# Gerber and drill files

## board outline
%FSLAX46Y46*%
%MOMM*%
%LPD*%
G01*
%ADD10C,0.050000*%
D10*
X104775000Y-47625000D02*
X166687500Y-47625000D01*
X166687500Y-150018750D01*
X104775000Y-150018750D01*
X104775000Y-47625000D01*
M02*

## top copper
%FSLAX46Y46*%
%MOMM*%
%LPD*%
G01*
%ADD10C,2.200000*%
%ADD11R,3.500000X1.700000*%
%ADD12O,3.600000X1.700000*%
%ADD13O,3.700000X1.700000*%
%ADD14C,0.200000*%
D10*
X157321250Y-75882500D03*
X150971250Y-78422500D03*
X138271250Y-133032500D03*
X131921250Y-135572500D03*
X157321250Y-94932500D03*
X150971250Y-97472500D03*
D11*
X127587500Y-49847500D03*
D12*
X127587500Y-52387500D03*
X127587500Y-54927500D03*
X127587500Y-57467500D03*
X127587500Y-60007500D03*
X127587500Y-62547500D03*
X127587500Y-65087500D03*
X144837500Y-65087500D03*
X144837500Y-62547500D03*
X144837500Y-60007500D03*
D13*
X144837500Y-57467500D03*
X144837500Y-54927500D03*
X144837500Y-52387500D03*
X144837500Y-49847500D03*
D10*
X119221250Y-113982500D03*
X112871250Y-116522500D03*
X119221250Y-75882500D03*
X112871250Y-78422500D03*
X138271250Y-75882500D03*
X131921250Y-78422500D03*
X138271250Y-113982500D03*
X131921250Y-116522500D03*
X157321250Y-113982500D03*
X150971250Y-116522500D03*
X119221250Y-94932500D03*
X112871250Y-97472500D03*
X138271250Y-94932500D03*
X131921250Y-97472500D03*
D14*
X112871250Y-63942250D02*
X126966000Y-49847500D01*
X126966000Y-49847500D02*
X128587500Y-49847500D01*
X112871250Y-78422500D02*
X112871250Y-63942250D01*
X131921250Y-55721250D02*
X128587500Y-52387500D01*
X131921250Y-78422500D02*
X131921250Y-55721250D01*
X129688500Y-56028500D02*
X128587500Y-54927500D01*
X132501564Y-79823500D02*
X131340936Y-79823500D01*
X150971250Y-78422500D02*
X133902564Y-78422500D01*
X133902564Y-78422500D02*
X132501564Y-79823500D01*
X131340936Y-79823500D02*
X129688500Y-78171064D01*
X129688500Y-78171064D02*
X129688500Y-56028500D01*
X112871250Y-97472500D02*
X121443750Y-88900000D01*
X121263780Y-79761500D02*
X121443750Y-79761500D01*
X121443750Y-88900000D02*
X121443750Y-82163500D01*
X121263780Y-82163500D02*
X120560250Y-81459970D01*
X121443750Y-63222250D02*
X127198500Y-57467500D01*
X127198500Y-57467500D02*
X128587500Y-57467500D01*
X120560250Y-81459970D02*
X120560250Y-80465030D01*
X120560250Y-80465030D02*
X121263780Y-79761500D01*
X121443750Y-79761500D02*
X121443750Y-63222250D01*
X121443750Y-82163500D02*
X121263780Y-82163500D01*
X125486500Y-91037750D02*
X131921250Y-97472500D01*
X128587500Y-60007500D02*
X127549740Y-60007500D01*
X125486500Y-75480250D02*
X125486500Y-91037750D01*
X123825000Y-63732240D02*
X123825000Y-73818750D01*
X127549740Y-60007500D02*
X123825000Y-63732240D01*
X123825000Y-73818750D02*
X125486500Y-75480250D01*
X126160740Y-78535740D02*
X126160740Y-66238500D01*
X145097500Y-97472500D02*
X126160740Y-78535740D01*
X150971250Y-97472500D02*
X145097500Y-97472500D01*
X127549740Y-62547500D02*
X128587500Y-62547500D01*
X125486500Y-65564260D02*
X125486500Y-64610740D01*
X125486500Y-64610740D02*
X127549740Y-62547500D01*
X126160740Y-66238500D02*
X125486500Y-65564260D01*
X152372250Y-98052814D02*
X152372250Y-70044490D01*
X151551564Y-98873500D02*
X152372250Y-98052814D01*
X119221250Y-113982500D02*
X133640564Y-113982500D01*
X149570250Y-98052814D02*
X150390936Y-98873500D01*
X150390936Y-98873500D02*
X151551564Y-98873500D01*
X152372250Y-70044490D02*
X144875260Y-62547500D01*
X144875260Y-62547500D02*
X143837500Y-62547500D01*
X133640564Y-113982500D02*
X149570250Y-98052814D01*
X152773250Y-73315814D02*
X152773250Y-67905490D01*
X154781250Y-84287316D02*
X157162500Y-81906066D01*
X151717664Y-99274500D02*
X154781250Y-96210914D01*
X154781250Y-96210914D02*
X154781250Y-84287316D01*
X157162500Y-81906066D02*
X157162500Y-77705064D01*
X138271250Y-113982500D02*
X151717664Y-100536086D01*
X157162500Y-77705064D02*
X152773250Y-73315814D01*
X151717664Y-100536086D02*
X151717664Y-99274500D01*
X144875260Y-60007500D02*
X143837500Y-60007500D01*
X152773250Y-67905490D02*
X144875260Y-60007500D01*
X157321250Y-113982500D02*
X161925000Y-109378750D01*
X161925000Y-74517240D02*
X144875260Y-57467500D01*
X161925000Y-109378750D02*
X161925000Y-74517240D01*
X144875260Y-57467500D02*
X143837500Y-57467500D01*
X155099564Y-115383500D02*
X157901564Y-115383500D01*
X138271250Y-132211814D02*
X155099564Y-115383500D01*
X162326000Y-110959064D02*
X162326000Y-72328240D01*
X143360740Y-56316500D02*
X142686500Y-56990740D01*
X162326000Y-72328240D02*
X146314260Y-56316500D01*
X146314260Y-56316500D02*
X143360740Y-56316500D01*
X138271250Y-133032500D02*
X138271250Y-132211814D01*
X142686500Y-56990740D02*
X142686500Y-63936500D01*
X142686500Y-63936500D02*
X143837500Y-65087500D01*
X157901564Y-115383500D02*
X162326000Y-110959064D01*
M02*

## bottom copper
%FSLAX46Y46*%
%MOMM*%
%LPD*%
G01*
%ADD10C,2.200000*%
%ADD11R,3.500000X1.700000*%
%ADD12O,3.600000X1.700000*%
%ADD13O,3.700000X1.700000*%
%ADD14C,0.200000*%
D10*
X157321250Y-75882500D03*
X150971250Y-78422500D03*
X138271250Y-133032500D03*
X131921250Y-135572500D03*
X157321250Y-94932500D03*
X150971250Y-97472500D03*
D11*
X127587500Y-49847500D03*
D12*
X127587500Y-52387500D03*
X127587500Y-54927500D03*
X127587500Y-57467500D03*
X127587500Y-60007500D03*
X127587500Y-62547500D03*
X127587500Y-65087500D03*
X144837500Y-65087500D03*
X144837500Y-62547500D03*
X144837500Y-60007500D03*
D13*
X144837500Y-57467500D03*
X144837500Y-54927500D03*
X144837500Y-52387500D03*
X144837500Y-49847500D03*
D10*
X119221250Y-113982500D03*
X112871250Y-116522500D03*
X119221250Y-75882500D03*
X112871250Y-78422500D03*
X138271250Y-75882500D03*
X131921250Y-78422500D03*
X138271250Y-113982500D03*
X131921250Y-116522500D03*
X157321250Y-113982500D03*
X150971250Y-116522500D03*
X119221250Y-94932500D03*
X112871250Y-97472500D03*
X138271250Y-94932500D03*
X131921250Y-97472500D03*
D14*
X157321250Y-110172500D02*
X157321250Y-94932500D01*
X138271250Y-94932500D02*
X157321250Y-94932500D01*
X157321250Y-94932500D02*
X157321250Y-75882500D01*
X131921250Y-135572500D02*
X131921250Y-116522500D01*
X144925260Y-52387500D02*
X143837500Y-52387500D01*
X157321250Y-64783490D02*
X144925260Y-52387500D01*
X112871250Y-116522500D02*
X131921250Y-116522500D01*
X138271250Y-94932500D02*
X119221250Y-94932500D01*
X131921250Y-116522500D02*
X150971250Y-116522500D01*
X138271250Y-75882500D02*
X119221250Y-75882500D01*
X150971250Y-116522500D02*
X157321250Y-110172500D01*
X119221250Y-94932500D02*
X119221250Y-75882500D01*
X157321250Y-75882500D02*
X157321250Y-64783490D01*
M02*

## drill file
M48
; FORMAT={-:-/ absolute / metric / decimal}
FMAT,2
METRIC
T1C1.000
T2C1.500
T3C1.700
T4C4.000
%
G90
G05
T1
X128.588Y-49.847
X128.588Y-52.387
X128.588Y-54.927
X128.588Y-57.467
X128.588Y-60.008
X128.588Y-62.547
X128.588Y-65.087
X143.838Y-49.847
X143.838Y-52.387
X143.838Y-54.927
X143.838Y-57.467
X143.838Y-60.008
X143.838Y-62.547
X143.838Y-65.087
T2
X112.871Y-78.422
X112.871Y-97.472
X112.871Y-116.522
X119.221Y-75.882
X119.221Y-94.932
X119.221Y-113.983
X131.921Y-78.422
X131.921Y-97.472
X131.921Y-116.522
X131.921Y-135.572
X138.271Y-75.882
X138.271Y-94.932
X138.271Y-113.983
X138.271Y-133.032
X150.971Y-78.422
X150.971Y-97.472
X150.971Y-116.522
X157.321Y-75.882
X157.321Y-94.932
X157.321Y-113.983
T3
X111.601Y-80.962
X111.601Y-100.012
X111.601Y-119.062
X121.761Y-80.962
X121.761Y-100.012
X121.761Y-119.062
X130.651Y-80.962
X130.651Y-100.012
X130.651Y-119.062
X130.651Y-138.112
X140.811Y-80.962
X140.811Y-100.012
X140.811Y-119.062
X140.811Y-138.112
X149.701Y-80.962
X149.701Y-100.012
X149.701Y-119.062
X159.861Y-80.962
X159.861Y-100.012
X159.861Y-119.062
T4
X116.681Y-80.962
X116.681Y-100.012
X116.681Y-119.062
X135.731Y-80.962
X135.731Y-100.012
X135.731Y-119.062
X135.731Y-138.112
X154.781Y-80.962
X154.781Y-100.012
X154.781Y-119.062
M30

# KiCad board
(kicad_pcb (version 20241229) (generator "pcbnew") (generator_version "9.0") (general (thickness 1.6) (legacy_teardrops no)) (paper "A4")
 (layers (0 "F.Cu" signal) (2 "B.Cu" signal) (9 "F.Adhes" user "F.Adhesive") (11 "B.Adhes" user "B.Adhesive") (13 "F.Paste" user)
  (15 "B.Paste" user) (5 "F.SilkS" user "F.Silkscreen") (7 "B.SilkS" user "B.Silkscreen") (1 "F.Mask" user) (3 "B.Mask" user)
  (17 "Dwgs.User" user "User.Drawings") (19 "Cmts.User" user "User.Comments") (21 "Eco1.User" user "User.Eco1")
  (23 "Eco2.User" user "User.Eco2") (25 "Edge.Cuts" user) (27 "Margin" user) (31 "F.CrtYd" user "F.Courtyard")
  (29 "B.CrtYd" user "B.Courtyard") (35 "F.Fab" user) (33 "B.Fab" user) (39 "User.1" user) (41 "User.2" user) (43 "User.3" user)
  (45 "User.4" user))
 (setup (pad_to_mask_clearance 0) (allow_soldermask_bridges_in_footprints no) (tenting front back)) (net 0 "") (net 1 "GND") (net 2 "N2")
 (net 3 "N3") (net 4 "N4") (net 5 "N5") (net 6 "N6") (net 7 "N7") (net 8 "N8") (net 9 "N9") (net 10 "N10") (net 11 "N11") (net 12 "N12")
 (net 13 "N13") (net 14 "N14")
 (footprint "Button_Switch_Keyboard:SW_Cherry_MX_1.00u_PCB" (layer "F.Cu") (at 157.32125 75.8825)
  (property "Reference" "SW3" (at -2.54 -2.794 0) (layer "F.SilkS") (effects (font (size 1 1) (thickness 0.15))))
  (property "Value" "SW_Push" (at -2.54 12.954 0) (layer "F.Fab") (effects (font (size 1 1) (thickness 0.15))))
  (pad "" np_thru_hole circle (at -7.62 5.08) (size 1.7 1.7) (drill 1.7) (layers "*.Cu" "*.Mask"))
  (pad "" np_thru_hole circle (at -2.54 5.08) (size 4 4) (drill 4) (layers "*.Cu" "*.Mask"))
  (pad "" np_thru_hole circle (at 2.54 5.08) (size 1.7 1.7) (drill 1.7) (layers "*.Cu" "*.Mask"))
  (pad "1" thru_hole circle (at 0 0) (size 2.2 2.2) (drill 1.5) (layers "*.Cu" "*.Mask") (remove_unused_layers no) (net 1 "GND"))
  (pad "2" thru_hole circle (at -6.35 2.54) (size 2.2 2.2) (drill 1.5) (layers "*.Cu" "*.Mask") (remove_unused_layers no) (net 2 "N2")))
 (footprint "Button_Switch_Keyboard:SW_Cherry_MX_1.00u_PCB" (layer "F.Cu") (at 138.27125 133.0325)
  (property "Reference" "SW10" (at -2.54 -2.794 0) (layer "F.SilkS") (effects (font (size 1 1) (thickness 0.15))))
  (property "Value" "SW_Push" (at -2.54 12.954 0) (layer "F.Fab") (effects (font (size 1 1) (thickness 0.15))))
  (pad "" np_thru_hole circle (at -7.62 5.08) (size 1.7 1.7) (drill 1.7) (layers "*.Cu" "*.Mask"))
  (pad "" np_thru_hole circle (at -2.54 5.08) (size 4 4) (drill 4) (layers "*.Cu" "*.Mask"))
  (pad "" np_thru_hole circle (at 2.54 5.08) (size 1.7 1.7) (drill 1.7) (layers "*.Cu" "*.Mask"))
  (pad "1" thru_hole circle (at 0 0) (size 2.2 2.2) (drill 1.5) (layers "*.Cu" "*.Mask") (remove_unused_layers no) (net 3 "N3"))
  (pad "2" thru_hole circle (at -6.35 2.54) (size 2.2 2.2) (drill 1.5) (layers "*.Cu" "*.Mask") (remove_unused_layers no) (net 1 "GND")))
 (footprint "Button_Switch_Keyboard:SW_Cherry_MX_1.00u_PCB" (layer "F.Cu") (at 157.32125 94.9325)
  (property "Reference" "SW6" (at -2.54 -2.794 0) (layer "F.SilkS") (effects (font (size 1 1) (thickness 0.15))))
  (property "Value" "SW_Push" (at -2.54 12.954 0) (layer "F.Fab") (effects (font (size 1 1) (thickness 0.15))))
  (pad "" np_thru_hole circle (at -7.62 5.08) (size 1.7 1.7) (drill 1.7) (layers "*.Cu" "*.Mask"))
  (pad "" np_thru_hole circle (at -2.54 5.08) (size 4 4) (drill 4) (layers "*.Cu" "*.Mask"))
  (pad "" np_thru_hole circle (at 2.54 5.08) (size 1.7 1.7) (drill 1.7) (layers "*.Cu" "*.Mask"))
  (pad "1" thru_hole circle (at 0 0) (size 2.2 2.2) (drill 1.5) (layers "*.Cu" "*.Mask") (remove_unused_layers no) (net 1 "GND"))
  (pad "2" thru_hole circle (at -6.35 2.54) (size 2.2 2.2) (drill 1.5) (layers "*.Cu" "*.Mask") (remove_unused_layers no) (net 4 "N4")))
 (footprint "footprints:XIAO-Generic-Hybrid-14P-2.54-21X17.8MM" (layer "F.Cu") (at 136.2125 57.4675)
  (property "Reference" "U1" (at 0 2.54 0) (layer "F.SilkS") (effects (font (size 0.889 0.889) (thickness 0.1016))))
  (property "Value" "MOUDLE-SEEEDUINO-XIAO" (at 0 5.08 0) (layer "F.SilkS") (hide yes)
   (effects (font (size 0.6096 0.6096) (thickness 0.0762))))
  (pad "1" thru_hole rect (at -7.625 -7.62) (size 3.5 1.7) (drill 1 (offset -1 0)) (layers "*.Cu" "*.Mask") (remove_unused_layers no)
   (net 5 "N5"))
  (pad "2" thru_hole oval (at -7.625 -5.08) (size 3.6 1.7) (drill 1 (offset -1 0)) (layers "*.Cu" "*.Mask") (remove_unused_layers no)
   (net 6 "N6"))
  (pad "3" thru_hole oval (at -7.625 -2.54) (size 3.6 1.7) (drill 1 (offset -1 0)) (layers "*.Cu" "*.Mask") (remove_unused_layers no)
   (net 2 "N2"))
  (pad "4" thru_hole oval (at -7.625 0) (size 3.6 1.7) (drill 1 (offset -1 0)) (layers "*.Cu" "*.Mask") (remove_unused_layers no)
   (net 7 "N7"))
  (pad "5" thru_hole oval (at -7.625 2.54) (size 3.6 1.7) (drill 1 (offset -1 0)) (layers "*.Cu" "*.Mask") (remove_unused_layers no)
   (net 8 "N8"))
  (pad "6" thru_hole oval (at -7.625 5.08 180) (size 3.6 1.7) (drill 1 (offset 1 0)) (layers "*.Cu" "*.Mask") (remove_unused_layers no)
   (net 4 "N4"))
  (pad "7" thru_hole oval (at -7.625 7.62) (size 3.6 1.7) (drill 1 (offset -1 0)) (layers "*.Cu" "*.Mask") (remove_unused_layers no)
   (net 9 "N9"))
  (pad "8" thru_hole oval (at 7.625 7.62) (size 3.6 1.7) (drill 1 (offset 1 0)) (layers "*.Cu" "*.Mask") (remove_unused_layers no)
   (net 3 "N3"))
  (pad "9" thru_hole oval (at 7.625 5.08) (size 3.6 1.7) (drill 1 (offset 1 0)) (layers "*.Cu" "*.Mask") (remove_unused_layers no)
   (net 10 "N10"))
  (pad "10" thru_hole oval (at 7.625 2.54) (size 3.6 1.7) (drill 1 (offset 1 0)) (layers "*.Cu" "*.Mask") (remove_unused_layers no)
   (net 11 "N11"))
  (pad "11" thru_hole oval (at 7.625 0) (size 3.7 1.7) (drill 1 (offset 1 0)) (layers "*.Cu" "*.Mask") (remove_unused_layers no)
   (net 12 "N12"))
  (pad "12" thru_hole oval (at 7.625 -2.54) (size 3.7 1.7) (drill 1 (offset 1 0)) (layers "*.Cu" "*.Mask") (remove_unused_layers no)
   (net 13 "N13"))
  (pad "13" thru_hole oval (at 7.625 -5.08) (size 3.7 1.7) (drill 1 (offset 1 0)) (layers "*.Cu" "*.Mask") (remove_unused_layers no)
   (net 1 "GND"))
  (pad "14" thru_hole oval (at 7.625 -7.62) (size 3.7 1.7) (drill 1 (offset 1 0)) (layers "*.Cu" "*.Mask") (remove_unused_layers no)
   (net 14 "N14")))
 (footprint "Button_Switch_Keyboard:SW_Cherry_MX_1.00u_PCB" (layer "F.Cu") (at 119.22125 113.9825)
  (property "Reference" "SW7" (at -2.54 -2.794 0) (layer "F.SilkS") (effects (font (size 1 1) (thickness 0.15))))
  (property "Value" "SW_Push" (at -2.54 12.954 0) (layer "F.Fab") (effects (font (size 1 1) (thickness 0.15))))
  (pad "" np_thru_hole circle (at -7.62 5.08) (size 1.7 1.7) (drill 1.7) (layers "*.Cu" "*.Mask"))
  (pad "" np_thru_hole circle (at -2.54 5.08) (size 4 4) (drill 4) (layers "*.Cu" "*.Mask"))
  (pad "" np_thru_hole circle (at 2.54 5.08) (size 1.7 1.7) (drill 1.7) (layers "*.Cu" "*.Mask"))
  (pad "1" thru_hole circle (at 0 0) (size 2.2 2.2) (drill 1.5) (layers "*.Cu" "*.Mask") (remove_unused_layers no) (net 10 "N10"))
  (pad "2" thru_hole circle (at -6.35 2.54) (size 2.2 2.2) (drill 1.5) (layers "*.Cu" "*.Mask") (remove_unused_layers no) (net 1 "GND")))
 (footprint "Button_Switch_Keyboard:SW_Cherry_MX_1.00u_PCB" (layer "F.Cu") (at 119.22125 75.8825)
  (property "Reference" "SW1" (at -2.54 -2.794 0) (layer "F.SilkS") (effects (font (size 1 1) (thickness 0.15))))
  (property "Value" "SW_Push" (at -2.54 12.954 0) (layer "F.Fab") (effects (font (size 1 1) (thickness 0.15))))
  (pad "" np_thru_hole circle (at -7.62 5.08) (size 1.7 1.7) (drill 1.7) (layers "*.Cu" "*.Mask"))
  (pad "" np_thru_hole circle (at -2.54 5.08) (size 4 4) (drill 4) (layers "*.Cu" "*.Mask"))
  (pad "" np_thru_hole circle (at 2.54 5.08) (size 1.7 1.7) (drill 1.7) (layers "*.Cu" "*.Mask"))
  (pad "1" thru_hole circle (at 0 0) (size 2.2 2.2) (drill 1.5) (layers "*.Cu" "*.Mask") (remove_unused_layers no) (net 1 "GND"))
  (pad "2" thru_hole circle (at -6.35 2.54) (size 2.2 2.2) (drill 1.5) (layers "*.Cu" "*.Mask") (remove_unused_layers no) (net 5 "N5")))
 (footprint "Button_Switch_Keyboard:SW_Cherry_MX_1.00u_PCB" (layer "F.Cu") (at 138.27125 75.8825)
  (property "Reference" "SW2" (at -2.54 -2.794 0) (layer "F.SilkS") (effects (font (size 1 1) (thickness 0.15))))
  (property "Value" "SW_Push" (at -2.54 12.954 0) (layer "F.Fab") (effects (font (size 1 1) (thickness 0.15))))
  (pad "" np_thru_hole circle (at -7.62 5.08) (size 1.7 1.7) (drill 1.7) (layers "*.Cu" "*.Mask"))
  (pad "" np_thru_hole circle (at -2.54 5.08) (size 4 4) (drill 4) (layers "*.Cu" "*.Mask"))
  (pad "" np_thru_hole circle (at 2.54 5.08) (size 1.7 1.7) (drill 1.7) (layers "*.Cu" "*.Mask"))
  (pad "1" thru_hole circle (at 0 0) (size 2.2 2.2) (drill 1.5) (layers "*.Cu" "*.Mask") (remove_unused_layers no) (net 1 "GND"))
  (pad "2" thru_hole circle (at -6.35 2.54) (size 2.2 2.2) (drill 1.5) (layers "*.Cu" "*.Mask") (remove_unused_layers no) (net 6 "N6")))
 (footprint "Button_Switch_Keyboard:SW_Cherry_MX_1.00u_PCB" (layer "F.Cu") (at 138.27125 113.9825)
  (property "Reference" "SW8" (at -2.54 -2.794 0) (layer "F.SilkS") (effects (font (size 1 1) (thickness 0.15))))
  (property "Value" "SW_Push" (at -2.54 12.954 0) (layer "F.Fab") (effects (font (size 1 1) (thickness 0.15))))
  (pad "" np_thru_hole circle (at -7.62 5.08) (size 1.7 1.7) (drill 1.7) (layers "*.Cu" "*.Mask"))
  (pad "" np_thru_hole circle (at -2.54 5.08) (size 4 4) (drill 4) (layers "*.Cu" "*.Mask"))
  (pad "" np_thru_hole circle (at 2.54 5.08) (size 1.7 1.7) (drill 1.7) (layers "*.Cu" "*.Mask"))
  (pad "1" thru_hole circle (at 0 0) (size 2.2 2.2) (drill 1.5) (layers "*.Cu" "*.Mask") (remove_unused_layers no) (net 11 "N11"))
  (pad "2" thru_hole circle (at -6.35 2.54) (size 2.2 2.2) (drill 1.5) (layers "*.Cu" "*.Mask") (remove_unused_layers no) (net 1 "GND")))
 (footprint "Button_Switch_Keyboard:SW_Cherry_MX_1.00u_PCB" (layer "F.Cu") (at 157.32125 113.9825)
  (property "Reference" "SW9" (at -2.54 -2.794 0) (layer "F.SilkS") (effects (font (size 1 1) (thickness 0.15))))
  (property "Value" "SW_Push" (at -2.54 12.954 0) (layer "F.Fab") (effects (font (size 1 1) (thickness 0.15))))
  (pad "" np_thru_hole circle (at -7.62 5.08) (size 1.7 1.7) (drill 1.7) (layers "*.Cu" "*.Mask"))
  (pad "" np_thru_hole circle (at -2.54 5.08) (size 4 4) (drill 4) (layers "*.Cu" "*.Mask"))
  (pad "" np_thru_hole circle (at 2.54 5.08) (size 1.7 1.7) (drill 1.7) (layers "*.Cu" "*.Mask"))
  (pad "1" thru_hole circle (at 0 0) (size 2.2 2.2) (drill 1.5) (layers "*.Cu" "*.Mask") (remove_unused_layers no) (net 12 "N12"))
  (pad "2" thru_hole circle (at -6.35 2.54) (size 2.2 2.2) (drill 1.5) (layers "*.Cu" "*.Mask") (remove_unused_layers no) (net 1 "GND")))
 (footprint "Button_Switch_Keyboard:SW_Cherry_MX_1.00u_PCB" (layer "F.Cu") (at 119.22125 94.9325)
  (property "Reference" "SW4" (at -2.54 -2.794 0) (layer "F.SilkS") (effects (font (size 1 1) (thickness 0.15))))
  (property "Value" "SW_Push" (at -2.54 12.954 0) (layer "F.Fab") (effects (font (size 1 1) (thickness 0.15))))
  (pad "" np_thru_hole circle (at -7.62 5.08) (size 1.7 1.7) (drill 1.7) (layers "*.Cu" "*.Mask"))
  (pad "" np_thru_hole circle (at -2.54 5.08) (size 4 4) (drill 4) (layers "*.Cu" "*.Mask"))
  (pad "" np_thru_hole circle (at 2.54 5.08) (size 1.7 1.7) (drill 1.7) (layers "*.Cu" "*.Mask"))
  (pad "1" thru_hole circle (at 0 0) (size 2.2 2.2) (drill 1.5) (layers "*.Cu" "*.Mask") (remove_unused_layers no) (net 1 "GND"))
  (pad "2" thru_hole circle (at -6.35 2.54) (size 2.2 2.2) (drill 1.5) (layers "*.Cu" "*.Mask") (remove_unused_layers no) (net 7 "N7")))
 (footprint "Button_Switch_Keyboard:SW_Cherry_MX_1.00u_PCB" (layer "F.Cu") (at 138.27125 94.9325)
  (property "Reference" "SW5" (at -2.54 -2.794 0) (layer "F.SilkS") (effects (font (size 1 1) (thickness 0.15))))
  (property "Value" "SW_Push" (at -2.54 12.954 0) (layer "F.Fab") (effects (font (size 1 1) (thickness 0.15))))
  (pad "" np_thru_hole circle (at -7.62 5.08) (size 1.7 1.7) (drill 1.7) (layers "*.Cu" "*.Mask"))
  (pad "" np_thru_hole circle (at -2.54 5.08) (size 4 4) (drill 4) (layers "*.Cu" "*.Mask"))
  (pad "" np_thru_hole circle (at 2.54 5.08) (size 1.7 1.7) (drill 1.7) (layers "*.Cu" "*.Mask"))
  (pad "1" thru_hole circle (at 0 0) (size 2.2 2.2) (drill 1.5) (layers "*.Cu" "*.Mask") (remove_unused_layers no) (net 1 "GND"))
  (pad "2" thru_hole circle (at -6.35 2.54) (size 2.2 2.2) (drill 1.5) (layers "*.Cu" "*.Mask") (remove_unused_layers no) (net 8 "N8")))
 (gr_rect (start 104.775 47.625) (end 166.6875 150.01875) (stroke (width 0.05) (type default)) (fill no) (layer "Edge.Cuts"))
 (segment (start 112.87125 63.94225) (end 126.966 49.8475) (width 0.2) (layer "F.Cu") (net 5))
 (segment (start 126.966 49.8475) (end 128.5875 49.8475) (width 0.2) (layer "F.Cu") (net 5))
 (segment (start 112.87125 78.4225) (end 112.87125 63.94225) (width 0.2) (layer "F.Cu") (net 5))
 (segment (start 157.32125 110.1725) (end 157.32125 94.9325) (width 0.2) (layer "B.Cu") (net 1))
 (segment (start 138.27125 94.9325) (end 157.32125 94.9325) (width 0.2) (layer "B.Cu") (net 1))
 (segment (start 157.32125 94.9325) (end 157.32125 75.8825) (width 0.2) (layer "B.Cu") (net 1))
 (segment (start 131.92125 135.5725) (end 131.92125 116.5225) (width 0.2) (layer "B.Cu") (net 1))
 (segment (start 144.92526 52.3875) (end 143.8375 52.3875) (width 0.2) (layer "B.Cu") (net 1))
 (segment (start 157.32125 64.78349) (end 144.92526 52.3875) (width 0.2) (layer "B.Cu") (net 1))
 (segment (start 112.87125 116.5225) (end 131.92125 116.5225) (width 0.2) (layer "B.Cu") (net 1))
 (segment (start 138.27125 94.9325) (end 119.22125 94.9325) (width 0.2) (layer "B.Cu") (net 1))
 (segment (start 131.92125 116.5225) (end 150.97125 116.5225) (width 0.2) (layer "B.Cu") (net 1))
 (segment (start 138.27125 75.8825) (end 119.22125 75.8825) (width 0.2) (layer "B.Cu") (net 1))
 (segment (start 150.97125 116.5225) (end 157.32125 110.1725) (width 0.2) (layer "B.Cu") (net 1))
 (segment (start 119.22125 94.9325) (end 119.22125 75.8825) (width 0.2) (layer "B.Cu") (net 1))
 (segment (start 157.32125 75.8825) (end 157.32125 64.78349) (width 0.2) (layer "B.Cu") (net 1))
 (segment (start 131.92125 55.72125) (end 128.5875 52.3875) (width 0.2) (layer "F.Cu") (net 6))
 (segment (start 131.92125 78.4225) (end 131.92125 55.72125) (width 0.2) (layer "F.Cu") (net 6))
 (segment (start 129.6885 56.0285) (end 128.5875 54.9275) (width 0.2) (layer "F.Cu") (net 2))
 (segment (start 132.501564 79.8235) (end 131.340936 79.8235) (width 0.2) (layer "F.Cu") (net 2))
 (segment (start 150.97125 78.4225) (end 133.902564 78.4225) (width 0.2) (layer "F.Cu") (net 2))
 (segment (start 133.902564 78.4225) (end 132.501564 79.8235) (width 0.2) (layer "F.Cu") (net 2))
 (segment (start 131.340936 79.8235) (end 129.6885 78.171064) (width 0.2) (layer "F.Cu") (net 2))
 (segment (start 129.6885 78.171064) (end 129.6885 56.0285) (width 0.2) (layer "F.Cu") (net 2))
 (segment (start 112.87125 97.4725) (end 121.44375 88.9) (width 0.2) (layer "F.Cu") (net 7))
 (segment (start 121.26378 79.7615) (end 121.44375 79.7615) (width 0.2) (layer "F.Cu") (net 7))
 (segment (start 121.44375 88.9) (end 121.44375 82.1635) (width 0.2) (layer "F.Cu") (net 7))
 (segment (start 121.26378 82.1635) (end 120.56025 81.45997) (width 0.2) (layer "F.Cu") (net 7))
 (segment (start 121.44375 63.22225) (end 127.1985 57.4675) (width 0.2) (layer "F.Cu") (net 7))
 (segment (start 127.1985 57.4675) (end 128.5875 57.4675) (width 0.2) (layer "F.Cu") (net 7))
 (segment (start 120.56025 81.45997) (end 120.56025 80.46503) (width 0.2) (layer "F.Cu") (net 7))
 (segment (start 120.56025 80.46503) (end 121.26378 79.7615) (width 0.2) (layer "F.Cu") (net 7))
 (segment (start 121.44375 79.7615) (end 121.44375 63.22225) (width 0.2) (layer "F.Cu") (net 7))
 (segment (start 121.44375 82.1635) (end 121.26378 82.1635) (width 0.2) (layer "F.Cu") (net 7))
 (segment (start 125.4865 91.03775) (end 131.92125 97.4725) (width 0.2) (layer "F.Cu") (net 8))
 (segment (start 128.5875 60.0075) (end 127.54974 60.0075) (width 0.2) (layer "F.Cu") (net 8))
 (segment (start 125.4865 75.48025) (end 125.4865 91.03775) (width 0.2) (layer "F.Cu") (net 8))
 (segment (start 123.825 63.73224) (end 123.825 73.81875) (width 0.2) (layer "F.Cu") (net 8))
 (segment (start 127.54974 60.0075) (end 123.825 63.73224) (width 0.2) (layer "F.Cu") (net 8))
 (segment (start 123.825 73.81875) (end 125.4865 75.48025) (width 0.2) (layer "F.Cu") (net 8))
 (segment (start 126.16074 78.53574) (end 126.16074 66.2385) (width 0.2) (layer "F.Cu") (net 4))
 (segment (start 145.0975 97.4725) (end 126.16074 78.53574) (width 0.2) (layer "F.Cu") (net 4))
 (segment (start 150.97125 97.4725) (end 145.0975 97.4725) (width 0.2) (layer "F.Cu") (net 4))
 (segment (start 127.54974 62.5475) (end 128.5875 62.5475) (width 0.2) (layer "F.Cu") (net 4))
 (segment (start 125.4865 65.56426) (end 125.4865 64.61074) (width 0.2) (layer "F.Cu") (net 4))
 (segment (start 125.4865 64.61074) (end 127.54974 62.5475) (width 0.2) (layer "F.Cu") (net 4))
 (segment (start 126.16074 66.2385) (end 125.4865 65.56426) (width 0.2) (layer "F.Cu") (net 4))
 (segment (start 152.37225 98.052814) (end 152.37225 70.04449) (width 0.2) (layer "F.Cu") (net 10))
 (segment (start 151.551564 98.8735) (end 152.37225 98.052814) (width 0.2) (layer "F.Cu") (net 10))
 (segment (start 119.22125 113.9825) (end 133.640564 113.9825) (width 0.2) (layer "F.Cu") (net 10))
 (segment (start 149.57025 98.052814) (end 150.390936 98.8735) (width 0.2) (layer "F.Cu") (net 10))
 (segment (start 150.390936 98.8735) (end 151.551564 98.8735) (width 0.2) (layer "F.Cu") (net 10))
 (segment (start 152.37225 70.04449) (end 144.87526 62.5475) (width 0.2) (layer "F.Cu") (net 10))
 (segment (start 144.87526 62.5475) (end 143.8375 62.5475) (width 0.2) (layer "F.Cu") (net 10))
 (segment (start 133.640564 113.9825) (end 149.57025 98.052814) (width 0.2) (layer "F.Cu") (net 10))
 (segment (start 152.77325 73.315814) (end 152.77325 67.90549) (width 0.2) (layer "F.Cu") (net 11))
 (segment (start 154.78125 84.287316) (end 157.1625 81.906066) (width 0.2) (layer "F.Cu") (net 11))
 (segment (start 151.717664 99.2745) (end 154.78125 96.210914) (width 0.2) (layer "F.Cu") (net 11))
 (segment (start 154.78125 96.210914) (end 154.78125 84.287316) (width 0.2) (layer "F.Cu") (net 11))
 (segment (start 157.1625 81.906066) (end 157.1625 77.705064) (width 0.2) (layer "F.Cu") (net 11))
 (segment (start 138.27125 113.9825) (end 151.717664 100.536086) (width 0.2) (layer "F.Cu") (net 11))
 (segment (start 157.1625 77.705064) (end 152.77325 73.315814) (width 0.2) (layer "F.Cu") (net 11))
 (segment (start 151.717664 100.536086) (end 151.717664 99.2745) (width 0.2) (layer "F.Cu") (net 11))
 (segment (start 144.87526 60.0075) (end 143.8375 60.0075) (width 0.2) (layer "F.Cu") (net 11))
 (segment (start 152.77325 67.90549) (end 144.87526 60.0075) (width 0.2) (layer "F.Cu") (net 11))
 (segment (start 157.32125 113.9825) (end 161.925 109.37875) (width 0.2) (layer "F.Cu") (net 12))
 (segment (start 161.925 74.51724) (end 144.87526 57.4675) (width 0.2) (layer "F.Cu") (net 12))
 (segment (start 161.925 109.37875) (end 161.925 74.51724) (width 0.2) (layer "F.Cu") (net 12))
 (segment (start 144.87526 57.4675) (end 143.8375 57.4675) (width 0.2) (layer "F.Cu") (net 12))
 (segment (start 155.099564 115.3835) (end 157.901564 115.3835) (width 0.2) (layer "F.Cu") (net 3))
 (segment (start 138.27125 132.211814) (end 155.099564 115.3835) (width 0.2) (layer "F.Cu") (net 3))
 (segment (start 162.326 110.959064) (end 162.326 72.32824) (width 0.2) (layer "F.Cu") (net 3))
 (segment (start 143.36074 56.3165) (end 142.6865 56.99074) (width 0.2) (layer "F.Cu") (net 3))
 (segment (start 162.326 72.32824) (end 146.31426 56.3165) (width 0.2) (layer "F.Cu") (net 3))
 (segment (start 146.31426 56.3165) (end 143.36074 56.3165) (width 0.2) (layer "F.Cu") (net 3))
 (segment (start 138.27125 133.0325) (end 138.27125 132.211814) (width 0.2) (layer "F.Cu") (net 3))
 (segment (start 142.6865 56.99074) (end 142.6865 63.9365) (width 0.2) (layer "F.Cu") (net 3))
 (segment (start 142.6865 63.9365) (end 143.8375 65.0875) (width 0.2) (layer "F.Cu") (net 3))
 (segment (start 157.901564 115.3835) (end 162.326 110.959064) (width 0.2) (layer "F.Cu") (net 3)))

